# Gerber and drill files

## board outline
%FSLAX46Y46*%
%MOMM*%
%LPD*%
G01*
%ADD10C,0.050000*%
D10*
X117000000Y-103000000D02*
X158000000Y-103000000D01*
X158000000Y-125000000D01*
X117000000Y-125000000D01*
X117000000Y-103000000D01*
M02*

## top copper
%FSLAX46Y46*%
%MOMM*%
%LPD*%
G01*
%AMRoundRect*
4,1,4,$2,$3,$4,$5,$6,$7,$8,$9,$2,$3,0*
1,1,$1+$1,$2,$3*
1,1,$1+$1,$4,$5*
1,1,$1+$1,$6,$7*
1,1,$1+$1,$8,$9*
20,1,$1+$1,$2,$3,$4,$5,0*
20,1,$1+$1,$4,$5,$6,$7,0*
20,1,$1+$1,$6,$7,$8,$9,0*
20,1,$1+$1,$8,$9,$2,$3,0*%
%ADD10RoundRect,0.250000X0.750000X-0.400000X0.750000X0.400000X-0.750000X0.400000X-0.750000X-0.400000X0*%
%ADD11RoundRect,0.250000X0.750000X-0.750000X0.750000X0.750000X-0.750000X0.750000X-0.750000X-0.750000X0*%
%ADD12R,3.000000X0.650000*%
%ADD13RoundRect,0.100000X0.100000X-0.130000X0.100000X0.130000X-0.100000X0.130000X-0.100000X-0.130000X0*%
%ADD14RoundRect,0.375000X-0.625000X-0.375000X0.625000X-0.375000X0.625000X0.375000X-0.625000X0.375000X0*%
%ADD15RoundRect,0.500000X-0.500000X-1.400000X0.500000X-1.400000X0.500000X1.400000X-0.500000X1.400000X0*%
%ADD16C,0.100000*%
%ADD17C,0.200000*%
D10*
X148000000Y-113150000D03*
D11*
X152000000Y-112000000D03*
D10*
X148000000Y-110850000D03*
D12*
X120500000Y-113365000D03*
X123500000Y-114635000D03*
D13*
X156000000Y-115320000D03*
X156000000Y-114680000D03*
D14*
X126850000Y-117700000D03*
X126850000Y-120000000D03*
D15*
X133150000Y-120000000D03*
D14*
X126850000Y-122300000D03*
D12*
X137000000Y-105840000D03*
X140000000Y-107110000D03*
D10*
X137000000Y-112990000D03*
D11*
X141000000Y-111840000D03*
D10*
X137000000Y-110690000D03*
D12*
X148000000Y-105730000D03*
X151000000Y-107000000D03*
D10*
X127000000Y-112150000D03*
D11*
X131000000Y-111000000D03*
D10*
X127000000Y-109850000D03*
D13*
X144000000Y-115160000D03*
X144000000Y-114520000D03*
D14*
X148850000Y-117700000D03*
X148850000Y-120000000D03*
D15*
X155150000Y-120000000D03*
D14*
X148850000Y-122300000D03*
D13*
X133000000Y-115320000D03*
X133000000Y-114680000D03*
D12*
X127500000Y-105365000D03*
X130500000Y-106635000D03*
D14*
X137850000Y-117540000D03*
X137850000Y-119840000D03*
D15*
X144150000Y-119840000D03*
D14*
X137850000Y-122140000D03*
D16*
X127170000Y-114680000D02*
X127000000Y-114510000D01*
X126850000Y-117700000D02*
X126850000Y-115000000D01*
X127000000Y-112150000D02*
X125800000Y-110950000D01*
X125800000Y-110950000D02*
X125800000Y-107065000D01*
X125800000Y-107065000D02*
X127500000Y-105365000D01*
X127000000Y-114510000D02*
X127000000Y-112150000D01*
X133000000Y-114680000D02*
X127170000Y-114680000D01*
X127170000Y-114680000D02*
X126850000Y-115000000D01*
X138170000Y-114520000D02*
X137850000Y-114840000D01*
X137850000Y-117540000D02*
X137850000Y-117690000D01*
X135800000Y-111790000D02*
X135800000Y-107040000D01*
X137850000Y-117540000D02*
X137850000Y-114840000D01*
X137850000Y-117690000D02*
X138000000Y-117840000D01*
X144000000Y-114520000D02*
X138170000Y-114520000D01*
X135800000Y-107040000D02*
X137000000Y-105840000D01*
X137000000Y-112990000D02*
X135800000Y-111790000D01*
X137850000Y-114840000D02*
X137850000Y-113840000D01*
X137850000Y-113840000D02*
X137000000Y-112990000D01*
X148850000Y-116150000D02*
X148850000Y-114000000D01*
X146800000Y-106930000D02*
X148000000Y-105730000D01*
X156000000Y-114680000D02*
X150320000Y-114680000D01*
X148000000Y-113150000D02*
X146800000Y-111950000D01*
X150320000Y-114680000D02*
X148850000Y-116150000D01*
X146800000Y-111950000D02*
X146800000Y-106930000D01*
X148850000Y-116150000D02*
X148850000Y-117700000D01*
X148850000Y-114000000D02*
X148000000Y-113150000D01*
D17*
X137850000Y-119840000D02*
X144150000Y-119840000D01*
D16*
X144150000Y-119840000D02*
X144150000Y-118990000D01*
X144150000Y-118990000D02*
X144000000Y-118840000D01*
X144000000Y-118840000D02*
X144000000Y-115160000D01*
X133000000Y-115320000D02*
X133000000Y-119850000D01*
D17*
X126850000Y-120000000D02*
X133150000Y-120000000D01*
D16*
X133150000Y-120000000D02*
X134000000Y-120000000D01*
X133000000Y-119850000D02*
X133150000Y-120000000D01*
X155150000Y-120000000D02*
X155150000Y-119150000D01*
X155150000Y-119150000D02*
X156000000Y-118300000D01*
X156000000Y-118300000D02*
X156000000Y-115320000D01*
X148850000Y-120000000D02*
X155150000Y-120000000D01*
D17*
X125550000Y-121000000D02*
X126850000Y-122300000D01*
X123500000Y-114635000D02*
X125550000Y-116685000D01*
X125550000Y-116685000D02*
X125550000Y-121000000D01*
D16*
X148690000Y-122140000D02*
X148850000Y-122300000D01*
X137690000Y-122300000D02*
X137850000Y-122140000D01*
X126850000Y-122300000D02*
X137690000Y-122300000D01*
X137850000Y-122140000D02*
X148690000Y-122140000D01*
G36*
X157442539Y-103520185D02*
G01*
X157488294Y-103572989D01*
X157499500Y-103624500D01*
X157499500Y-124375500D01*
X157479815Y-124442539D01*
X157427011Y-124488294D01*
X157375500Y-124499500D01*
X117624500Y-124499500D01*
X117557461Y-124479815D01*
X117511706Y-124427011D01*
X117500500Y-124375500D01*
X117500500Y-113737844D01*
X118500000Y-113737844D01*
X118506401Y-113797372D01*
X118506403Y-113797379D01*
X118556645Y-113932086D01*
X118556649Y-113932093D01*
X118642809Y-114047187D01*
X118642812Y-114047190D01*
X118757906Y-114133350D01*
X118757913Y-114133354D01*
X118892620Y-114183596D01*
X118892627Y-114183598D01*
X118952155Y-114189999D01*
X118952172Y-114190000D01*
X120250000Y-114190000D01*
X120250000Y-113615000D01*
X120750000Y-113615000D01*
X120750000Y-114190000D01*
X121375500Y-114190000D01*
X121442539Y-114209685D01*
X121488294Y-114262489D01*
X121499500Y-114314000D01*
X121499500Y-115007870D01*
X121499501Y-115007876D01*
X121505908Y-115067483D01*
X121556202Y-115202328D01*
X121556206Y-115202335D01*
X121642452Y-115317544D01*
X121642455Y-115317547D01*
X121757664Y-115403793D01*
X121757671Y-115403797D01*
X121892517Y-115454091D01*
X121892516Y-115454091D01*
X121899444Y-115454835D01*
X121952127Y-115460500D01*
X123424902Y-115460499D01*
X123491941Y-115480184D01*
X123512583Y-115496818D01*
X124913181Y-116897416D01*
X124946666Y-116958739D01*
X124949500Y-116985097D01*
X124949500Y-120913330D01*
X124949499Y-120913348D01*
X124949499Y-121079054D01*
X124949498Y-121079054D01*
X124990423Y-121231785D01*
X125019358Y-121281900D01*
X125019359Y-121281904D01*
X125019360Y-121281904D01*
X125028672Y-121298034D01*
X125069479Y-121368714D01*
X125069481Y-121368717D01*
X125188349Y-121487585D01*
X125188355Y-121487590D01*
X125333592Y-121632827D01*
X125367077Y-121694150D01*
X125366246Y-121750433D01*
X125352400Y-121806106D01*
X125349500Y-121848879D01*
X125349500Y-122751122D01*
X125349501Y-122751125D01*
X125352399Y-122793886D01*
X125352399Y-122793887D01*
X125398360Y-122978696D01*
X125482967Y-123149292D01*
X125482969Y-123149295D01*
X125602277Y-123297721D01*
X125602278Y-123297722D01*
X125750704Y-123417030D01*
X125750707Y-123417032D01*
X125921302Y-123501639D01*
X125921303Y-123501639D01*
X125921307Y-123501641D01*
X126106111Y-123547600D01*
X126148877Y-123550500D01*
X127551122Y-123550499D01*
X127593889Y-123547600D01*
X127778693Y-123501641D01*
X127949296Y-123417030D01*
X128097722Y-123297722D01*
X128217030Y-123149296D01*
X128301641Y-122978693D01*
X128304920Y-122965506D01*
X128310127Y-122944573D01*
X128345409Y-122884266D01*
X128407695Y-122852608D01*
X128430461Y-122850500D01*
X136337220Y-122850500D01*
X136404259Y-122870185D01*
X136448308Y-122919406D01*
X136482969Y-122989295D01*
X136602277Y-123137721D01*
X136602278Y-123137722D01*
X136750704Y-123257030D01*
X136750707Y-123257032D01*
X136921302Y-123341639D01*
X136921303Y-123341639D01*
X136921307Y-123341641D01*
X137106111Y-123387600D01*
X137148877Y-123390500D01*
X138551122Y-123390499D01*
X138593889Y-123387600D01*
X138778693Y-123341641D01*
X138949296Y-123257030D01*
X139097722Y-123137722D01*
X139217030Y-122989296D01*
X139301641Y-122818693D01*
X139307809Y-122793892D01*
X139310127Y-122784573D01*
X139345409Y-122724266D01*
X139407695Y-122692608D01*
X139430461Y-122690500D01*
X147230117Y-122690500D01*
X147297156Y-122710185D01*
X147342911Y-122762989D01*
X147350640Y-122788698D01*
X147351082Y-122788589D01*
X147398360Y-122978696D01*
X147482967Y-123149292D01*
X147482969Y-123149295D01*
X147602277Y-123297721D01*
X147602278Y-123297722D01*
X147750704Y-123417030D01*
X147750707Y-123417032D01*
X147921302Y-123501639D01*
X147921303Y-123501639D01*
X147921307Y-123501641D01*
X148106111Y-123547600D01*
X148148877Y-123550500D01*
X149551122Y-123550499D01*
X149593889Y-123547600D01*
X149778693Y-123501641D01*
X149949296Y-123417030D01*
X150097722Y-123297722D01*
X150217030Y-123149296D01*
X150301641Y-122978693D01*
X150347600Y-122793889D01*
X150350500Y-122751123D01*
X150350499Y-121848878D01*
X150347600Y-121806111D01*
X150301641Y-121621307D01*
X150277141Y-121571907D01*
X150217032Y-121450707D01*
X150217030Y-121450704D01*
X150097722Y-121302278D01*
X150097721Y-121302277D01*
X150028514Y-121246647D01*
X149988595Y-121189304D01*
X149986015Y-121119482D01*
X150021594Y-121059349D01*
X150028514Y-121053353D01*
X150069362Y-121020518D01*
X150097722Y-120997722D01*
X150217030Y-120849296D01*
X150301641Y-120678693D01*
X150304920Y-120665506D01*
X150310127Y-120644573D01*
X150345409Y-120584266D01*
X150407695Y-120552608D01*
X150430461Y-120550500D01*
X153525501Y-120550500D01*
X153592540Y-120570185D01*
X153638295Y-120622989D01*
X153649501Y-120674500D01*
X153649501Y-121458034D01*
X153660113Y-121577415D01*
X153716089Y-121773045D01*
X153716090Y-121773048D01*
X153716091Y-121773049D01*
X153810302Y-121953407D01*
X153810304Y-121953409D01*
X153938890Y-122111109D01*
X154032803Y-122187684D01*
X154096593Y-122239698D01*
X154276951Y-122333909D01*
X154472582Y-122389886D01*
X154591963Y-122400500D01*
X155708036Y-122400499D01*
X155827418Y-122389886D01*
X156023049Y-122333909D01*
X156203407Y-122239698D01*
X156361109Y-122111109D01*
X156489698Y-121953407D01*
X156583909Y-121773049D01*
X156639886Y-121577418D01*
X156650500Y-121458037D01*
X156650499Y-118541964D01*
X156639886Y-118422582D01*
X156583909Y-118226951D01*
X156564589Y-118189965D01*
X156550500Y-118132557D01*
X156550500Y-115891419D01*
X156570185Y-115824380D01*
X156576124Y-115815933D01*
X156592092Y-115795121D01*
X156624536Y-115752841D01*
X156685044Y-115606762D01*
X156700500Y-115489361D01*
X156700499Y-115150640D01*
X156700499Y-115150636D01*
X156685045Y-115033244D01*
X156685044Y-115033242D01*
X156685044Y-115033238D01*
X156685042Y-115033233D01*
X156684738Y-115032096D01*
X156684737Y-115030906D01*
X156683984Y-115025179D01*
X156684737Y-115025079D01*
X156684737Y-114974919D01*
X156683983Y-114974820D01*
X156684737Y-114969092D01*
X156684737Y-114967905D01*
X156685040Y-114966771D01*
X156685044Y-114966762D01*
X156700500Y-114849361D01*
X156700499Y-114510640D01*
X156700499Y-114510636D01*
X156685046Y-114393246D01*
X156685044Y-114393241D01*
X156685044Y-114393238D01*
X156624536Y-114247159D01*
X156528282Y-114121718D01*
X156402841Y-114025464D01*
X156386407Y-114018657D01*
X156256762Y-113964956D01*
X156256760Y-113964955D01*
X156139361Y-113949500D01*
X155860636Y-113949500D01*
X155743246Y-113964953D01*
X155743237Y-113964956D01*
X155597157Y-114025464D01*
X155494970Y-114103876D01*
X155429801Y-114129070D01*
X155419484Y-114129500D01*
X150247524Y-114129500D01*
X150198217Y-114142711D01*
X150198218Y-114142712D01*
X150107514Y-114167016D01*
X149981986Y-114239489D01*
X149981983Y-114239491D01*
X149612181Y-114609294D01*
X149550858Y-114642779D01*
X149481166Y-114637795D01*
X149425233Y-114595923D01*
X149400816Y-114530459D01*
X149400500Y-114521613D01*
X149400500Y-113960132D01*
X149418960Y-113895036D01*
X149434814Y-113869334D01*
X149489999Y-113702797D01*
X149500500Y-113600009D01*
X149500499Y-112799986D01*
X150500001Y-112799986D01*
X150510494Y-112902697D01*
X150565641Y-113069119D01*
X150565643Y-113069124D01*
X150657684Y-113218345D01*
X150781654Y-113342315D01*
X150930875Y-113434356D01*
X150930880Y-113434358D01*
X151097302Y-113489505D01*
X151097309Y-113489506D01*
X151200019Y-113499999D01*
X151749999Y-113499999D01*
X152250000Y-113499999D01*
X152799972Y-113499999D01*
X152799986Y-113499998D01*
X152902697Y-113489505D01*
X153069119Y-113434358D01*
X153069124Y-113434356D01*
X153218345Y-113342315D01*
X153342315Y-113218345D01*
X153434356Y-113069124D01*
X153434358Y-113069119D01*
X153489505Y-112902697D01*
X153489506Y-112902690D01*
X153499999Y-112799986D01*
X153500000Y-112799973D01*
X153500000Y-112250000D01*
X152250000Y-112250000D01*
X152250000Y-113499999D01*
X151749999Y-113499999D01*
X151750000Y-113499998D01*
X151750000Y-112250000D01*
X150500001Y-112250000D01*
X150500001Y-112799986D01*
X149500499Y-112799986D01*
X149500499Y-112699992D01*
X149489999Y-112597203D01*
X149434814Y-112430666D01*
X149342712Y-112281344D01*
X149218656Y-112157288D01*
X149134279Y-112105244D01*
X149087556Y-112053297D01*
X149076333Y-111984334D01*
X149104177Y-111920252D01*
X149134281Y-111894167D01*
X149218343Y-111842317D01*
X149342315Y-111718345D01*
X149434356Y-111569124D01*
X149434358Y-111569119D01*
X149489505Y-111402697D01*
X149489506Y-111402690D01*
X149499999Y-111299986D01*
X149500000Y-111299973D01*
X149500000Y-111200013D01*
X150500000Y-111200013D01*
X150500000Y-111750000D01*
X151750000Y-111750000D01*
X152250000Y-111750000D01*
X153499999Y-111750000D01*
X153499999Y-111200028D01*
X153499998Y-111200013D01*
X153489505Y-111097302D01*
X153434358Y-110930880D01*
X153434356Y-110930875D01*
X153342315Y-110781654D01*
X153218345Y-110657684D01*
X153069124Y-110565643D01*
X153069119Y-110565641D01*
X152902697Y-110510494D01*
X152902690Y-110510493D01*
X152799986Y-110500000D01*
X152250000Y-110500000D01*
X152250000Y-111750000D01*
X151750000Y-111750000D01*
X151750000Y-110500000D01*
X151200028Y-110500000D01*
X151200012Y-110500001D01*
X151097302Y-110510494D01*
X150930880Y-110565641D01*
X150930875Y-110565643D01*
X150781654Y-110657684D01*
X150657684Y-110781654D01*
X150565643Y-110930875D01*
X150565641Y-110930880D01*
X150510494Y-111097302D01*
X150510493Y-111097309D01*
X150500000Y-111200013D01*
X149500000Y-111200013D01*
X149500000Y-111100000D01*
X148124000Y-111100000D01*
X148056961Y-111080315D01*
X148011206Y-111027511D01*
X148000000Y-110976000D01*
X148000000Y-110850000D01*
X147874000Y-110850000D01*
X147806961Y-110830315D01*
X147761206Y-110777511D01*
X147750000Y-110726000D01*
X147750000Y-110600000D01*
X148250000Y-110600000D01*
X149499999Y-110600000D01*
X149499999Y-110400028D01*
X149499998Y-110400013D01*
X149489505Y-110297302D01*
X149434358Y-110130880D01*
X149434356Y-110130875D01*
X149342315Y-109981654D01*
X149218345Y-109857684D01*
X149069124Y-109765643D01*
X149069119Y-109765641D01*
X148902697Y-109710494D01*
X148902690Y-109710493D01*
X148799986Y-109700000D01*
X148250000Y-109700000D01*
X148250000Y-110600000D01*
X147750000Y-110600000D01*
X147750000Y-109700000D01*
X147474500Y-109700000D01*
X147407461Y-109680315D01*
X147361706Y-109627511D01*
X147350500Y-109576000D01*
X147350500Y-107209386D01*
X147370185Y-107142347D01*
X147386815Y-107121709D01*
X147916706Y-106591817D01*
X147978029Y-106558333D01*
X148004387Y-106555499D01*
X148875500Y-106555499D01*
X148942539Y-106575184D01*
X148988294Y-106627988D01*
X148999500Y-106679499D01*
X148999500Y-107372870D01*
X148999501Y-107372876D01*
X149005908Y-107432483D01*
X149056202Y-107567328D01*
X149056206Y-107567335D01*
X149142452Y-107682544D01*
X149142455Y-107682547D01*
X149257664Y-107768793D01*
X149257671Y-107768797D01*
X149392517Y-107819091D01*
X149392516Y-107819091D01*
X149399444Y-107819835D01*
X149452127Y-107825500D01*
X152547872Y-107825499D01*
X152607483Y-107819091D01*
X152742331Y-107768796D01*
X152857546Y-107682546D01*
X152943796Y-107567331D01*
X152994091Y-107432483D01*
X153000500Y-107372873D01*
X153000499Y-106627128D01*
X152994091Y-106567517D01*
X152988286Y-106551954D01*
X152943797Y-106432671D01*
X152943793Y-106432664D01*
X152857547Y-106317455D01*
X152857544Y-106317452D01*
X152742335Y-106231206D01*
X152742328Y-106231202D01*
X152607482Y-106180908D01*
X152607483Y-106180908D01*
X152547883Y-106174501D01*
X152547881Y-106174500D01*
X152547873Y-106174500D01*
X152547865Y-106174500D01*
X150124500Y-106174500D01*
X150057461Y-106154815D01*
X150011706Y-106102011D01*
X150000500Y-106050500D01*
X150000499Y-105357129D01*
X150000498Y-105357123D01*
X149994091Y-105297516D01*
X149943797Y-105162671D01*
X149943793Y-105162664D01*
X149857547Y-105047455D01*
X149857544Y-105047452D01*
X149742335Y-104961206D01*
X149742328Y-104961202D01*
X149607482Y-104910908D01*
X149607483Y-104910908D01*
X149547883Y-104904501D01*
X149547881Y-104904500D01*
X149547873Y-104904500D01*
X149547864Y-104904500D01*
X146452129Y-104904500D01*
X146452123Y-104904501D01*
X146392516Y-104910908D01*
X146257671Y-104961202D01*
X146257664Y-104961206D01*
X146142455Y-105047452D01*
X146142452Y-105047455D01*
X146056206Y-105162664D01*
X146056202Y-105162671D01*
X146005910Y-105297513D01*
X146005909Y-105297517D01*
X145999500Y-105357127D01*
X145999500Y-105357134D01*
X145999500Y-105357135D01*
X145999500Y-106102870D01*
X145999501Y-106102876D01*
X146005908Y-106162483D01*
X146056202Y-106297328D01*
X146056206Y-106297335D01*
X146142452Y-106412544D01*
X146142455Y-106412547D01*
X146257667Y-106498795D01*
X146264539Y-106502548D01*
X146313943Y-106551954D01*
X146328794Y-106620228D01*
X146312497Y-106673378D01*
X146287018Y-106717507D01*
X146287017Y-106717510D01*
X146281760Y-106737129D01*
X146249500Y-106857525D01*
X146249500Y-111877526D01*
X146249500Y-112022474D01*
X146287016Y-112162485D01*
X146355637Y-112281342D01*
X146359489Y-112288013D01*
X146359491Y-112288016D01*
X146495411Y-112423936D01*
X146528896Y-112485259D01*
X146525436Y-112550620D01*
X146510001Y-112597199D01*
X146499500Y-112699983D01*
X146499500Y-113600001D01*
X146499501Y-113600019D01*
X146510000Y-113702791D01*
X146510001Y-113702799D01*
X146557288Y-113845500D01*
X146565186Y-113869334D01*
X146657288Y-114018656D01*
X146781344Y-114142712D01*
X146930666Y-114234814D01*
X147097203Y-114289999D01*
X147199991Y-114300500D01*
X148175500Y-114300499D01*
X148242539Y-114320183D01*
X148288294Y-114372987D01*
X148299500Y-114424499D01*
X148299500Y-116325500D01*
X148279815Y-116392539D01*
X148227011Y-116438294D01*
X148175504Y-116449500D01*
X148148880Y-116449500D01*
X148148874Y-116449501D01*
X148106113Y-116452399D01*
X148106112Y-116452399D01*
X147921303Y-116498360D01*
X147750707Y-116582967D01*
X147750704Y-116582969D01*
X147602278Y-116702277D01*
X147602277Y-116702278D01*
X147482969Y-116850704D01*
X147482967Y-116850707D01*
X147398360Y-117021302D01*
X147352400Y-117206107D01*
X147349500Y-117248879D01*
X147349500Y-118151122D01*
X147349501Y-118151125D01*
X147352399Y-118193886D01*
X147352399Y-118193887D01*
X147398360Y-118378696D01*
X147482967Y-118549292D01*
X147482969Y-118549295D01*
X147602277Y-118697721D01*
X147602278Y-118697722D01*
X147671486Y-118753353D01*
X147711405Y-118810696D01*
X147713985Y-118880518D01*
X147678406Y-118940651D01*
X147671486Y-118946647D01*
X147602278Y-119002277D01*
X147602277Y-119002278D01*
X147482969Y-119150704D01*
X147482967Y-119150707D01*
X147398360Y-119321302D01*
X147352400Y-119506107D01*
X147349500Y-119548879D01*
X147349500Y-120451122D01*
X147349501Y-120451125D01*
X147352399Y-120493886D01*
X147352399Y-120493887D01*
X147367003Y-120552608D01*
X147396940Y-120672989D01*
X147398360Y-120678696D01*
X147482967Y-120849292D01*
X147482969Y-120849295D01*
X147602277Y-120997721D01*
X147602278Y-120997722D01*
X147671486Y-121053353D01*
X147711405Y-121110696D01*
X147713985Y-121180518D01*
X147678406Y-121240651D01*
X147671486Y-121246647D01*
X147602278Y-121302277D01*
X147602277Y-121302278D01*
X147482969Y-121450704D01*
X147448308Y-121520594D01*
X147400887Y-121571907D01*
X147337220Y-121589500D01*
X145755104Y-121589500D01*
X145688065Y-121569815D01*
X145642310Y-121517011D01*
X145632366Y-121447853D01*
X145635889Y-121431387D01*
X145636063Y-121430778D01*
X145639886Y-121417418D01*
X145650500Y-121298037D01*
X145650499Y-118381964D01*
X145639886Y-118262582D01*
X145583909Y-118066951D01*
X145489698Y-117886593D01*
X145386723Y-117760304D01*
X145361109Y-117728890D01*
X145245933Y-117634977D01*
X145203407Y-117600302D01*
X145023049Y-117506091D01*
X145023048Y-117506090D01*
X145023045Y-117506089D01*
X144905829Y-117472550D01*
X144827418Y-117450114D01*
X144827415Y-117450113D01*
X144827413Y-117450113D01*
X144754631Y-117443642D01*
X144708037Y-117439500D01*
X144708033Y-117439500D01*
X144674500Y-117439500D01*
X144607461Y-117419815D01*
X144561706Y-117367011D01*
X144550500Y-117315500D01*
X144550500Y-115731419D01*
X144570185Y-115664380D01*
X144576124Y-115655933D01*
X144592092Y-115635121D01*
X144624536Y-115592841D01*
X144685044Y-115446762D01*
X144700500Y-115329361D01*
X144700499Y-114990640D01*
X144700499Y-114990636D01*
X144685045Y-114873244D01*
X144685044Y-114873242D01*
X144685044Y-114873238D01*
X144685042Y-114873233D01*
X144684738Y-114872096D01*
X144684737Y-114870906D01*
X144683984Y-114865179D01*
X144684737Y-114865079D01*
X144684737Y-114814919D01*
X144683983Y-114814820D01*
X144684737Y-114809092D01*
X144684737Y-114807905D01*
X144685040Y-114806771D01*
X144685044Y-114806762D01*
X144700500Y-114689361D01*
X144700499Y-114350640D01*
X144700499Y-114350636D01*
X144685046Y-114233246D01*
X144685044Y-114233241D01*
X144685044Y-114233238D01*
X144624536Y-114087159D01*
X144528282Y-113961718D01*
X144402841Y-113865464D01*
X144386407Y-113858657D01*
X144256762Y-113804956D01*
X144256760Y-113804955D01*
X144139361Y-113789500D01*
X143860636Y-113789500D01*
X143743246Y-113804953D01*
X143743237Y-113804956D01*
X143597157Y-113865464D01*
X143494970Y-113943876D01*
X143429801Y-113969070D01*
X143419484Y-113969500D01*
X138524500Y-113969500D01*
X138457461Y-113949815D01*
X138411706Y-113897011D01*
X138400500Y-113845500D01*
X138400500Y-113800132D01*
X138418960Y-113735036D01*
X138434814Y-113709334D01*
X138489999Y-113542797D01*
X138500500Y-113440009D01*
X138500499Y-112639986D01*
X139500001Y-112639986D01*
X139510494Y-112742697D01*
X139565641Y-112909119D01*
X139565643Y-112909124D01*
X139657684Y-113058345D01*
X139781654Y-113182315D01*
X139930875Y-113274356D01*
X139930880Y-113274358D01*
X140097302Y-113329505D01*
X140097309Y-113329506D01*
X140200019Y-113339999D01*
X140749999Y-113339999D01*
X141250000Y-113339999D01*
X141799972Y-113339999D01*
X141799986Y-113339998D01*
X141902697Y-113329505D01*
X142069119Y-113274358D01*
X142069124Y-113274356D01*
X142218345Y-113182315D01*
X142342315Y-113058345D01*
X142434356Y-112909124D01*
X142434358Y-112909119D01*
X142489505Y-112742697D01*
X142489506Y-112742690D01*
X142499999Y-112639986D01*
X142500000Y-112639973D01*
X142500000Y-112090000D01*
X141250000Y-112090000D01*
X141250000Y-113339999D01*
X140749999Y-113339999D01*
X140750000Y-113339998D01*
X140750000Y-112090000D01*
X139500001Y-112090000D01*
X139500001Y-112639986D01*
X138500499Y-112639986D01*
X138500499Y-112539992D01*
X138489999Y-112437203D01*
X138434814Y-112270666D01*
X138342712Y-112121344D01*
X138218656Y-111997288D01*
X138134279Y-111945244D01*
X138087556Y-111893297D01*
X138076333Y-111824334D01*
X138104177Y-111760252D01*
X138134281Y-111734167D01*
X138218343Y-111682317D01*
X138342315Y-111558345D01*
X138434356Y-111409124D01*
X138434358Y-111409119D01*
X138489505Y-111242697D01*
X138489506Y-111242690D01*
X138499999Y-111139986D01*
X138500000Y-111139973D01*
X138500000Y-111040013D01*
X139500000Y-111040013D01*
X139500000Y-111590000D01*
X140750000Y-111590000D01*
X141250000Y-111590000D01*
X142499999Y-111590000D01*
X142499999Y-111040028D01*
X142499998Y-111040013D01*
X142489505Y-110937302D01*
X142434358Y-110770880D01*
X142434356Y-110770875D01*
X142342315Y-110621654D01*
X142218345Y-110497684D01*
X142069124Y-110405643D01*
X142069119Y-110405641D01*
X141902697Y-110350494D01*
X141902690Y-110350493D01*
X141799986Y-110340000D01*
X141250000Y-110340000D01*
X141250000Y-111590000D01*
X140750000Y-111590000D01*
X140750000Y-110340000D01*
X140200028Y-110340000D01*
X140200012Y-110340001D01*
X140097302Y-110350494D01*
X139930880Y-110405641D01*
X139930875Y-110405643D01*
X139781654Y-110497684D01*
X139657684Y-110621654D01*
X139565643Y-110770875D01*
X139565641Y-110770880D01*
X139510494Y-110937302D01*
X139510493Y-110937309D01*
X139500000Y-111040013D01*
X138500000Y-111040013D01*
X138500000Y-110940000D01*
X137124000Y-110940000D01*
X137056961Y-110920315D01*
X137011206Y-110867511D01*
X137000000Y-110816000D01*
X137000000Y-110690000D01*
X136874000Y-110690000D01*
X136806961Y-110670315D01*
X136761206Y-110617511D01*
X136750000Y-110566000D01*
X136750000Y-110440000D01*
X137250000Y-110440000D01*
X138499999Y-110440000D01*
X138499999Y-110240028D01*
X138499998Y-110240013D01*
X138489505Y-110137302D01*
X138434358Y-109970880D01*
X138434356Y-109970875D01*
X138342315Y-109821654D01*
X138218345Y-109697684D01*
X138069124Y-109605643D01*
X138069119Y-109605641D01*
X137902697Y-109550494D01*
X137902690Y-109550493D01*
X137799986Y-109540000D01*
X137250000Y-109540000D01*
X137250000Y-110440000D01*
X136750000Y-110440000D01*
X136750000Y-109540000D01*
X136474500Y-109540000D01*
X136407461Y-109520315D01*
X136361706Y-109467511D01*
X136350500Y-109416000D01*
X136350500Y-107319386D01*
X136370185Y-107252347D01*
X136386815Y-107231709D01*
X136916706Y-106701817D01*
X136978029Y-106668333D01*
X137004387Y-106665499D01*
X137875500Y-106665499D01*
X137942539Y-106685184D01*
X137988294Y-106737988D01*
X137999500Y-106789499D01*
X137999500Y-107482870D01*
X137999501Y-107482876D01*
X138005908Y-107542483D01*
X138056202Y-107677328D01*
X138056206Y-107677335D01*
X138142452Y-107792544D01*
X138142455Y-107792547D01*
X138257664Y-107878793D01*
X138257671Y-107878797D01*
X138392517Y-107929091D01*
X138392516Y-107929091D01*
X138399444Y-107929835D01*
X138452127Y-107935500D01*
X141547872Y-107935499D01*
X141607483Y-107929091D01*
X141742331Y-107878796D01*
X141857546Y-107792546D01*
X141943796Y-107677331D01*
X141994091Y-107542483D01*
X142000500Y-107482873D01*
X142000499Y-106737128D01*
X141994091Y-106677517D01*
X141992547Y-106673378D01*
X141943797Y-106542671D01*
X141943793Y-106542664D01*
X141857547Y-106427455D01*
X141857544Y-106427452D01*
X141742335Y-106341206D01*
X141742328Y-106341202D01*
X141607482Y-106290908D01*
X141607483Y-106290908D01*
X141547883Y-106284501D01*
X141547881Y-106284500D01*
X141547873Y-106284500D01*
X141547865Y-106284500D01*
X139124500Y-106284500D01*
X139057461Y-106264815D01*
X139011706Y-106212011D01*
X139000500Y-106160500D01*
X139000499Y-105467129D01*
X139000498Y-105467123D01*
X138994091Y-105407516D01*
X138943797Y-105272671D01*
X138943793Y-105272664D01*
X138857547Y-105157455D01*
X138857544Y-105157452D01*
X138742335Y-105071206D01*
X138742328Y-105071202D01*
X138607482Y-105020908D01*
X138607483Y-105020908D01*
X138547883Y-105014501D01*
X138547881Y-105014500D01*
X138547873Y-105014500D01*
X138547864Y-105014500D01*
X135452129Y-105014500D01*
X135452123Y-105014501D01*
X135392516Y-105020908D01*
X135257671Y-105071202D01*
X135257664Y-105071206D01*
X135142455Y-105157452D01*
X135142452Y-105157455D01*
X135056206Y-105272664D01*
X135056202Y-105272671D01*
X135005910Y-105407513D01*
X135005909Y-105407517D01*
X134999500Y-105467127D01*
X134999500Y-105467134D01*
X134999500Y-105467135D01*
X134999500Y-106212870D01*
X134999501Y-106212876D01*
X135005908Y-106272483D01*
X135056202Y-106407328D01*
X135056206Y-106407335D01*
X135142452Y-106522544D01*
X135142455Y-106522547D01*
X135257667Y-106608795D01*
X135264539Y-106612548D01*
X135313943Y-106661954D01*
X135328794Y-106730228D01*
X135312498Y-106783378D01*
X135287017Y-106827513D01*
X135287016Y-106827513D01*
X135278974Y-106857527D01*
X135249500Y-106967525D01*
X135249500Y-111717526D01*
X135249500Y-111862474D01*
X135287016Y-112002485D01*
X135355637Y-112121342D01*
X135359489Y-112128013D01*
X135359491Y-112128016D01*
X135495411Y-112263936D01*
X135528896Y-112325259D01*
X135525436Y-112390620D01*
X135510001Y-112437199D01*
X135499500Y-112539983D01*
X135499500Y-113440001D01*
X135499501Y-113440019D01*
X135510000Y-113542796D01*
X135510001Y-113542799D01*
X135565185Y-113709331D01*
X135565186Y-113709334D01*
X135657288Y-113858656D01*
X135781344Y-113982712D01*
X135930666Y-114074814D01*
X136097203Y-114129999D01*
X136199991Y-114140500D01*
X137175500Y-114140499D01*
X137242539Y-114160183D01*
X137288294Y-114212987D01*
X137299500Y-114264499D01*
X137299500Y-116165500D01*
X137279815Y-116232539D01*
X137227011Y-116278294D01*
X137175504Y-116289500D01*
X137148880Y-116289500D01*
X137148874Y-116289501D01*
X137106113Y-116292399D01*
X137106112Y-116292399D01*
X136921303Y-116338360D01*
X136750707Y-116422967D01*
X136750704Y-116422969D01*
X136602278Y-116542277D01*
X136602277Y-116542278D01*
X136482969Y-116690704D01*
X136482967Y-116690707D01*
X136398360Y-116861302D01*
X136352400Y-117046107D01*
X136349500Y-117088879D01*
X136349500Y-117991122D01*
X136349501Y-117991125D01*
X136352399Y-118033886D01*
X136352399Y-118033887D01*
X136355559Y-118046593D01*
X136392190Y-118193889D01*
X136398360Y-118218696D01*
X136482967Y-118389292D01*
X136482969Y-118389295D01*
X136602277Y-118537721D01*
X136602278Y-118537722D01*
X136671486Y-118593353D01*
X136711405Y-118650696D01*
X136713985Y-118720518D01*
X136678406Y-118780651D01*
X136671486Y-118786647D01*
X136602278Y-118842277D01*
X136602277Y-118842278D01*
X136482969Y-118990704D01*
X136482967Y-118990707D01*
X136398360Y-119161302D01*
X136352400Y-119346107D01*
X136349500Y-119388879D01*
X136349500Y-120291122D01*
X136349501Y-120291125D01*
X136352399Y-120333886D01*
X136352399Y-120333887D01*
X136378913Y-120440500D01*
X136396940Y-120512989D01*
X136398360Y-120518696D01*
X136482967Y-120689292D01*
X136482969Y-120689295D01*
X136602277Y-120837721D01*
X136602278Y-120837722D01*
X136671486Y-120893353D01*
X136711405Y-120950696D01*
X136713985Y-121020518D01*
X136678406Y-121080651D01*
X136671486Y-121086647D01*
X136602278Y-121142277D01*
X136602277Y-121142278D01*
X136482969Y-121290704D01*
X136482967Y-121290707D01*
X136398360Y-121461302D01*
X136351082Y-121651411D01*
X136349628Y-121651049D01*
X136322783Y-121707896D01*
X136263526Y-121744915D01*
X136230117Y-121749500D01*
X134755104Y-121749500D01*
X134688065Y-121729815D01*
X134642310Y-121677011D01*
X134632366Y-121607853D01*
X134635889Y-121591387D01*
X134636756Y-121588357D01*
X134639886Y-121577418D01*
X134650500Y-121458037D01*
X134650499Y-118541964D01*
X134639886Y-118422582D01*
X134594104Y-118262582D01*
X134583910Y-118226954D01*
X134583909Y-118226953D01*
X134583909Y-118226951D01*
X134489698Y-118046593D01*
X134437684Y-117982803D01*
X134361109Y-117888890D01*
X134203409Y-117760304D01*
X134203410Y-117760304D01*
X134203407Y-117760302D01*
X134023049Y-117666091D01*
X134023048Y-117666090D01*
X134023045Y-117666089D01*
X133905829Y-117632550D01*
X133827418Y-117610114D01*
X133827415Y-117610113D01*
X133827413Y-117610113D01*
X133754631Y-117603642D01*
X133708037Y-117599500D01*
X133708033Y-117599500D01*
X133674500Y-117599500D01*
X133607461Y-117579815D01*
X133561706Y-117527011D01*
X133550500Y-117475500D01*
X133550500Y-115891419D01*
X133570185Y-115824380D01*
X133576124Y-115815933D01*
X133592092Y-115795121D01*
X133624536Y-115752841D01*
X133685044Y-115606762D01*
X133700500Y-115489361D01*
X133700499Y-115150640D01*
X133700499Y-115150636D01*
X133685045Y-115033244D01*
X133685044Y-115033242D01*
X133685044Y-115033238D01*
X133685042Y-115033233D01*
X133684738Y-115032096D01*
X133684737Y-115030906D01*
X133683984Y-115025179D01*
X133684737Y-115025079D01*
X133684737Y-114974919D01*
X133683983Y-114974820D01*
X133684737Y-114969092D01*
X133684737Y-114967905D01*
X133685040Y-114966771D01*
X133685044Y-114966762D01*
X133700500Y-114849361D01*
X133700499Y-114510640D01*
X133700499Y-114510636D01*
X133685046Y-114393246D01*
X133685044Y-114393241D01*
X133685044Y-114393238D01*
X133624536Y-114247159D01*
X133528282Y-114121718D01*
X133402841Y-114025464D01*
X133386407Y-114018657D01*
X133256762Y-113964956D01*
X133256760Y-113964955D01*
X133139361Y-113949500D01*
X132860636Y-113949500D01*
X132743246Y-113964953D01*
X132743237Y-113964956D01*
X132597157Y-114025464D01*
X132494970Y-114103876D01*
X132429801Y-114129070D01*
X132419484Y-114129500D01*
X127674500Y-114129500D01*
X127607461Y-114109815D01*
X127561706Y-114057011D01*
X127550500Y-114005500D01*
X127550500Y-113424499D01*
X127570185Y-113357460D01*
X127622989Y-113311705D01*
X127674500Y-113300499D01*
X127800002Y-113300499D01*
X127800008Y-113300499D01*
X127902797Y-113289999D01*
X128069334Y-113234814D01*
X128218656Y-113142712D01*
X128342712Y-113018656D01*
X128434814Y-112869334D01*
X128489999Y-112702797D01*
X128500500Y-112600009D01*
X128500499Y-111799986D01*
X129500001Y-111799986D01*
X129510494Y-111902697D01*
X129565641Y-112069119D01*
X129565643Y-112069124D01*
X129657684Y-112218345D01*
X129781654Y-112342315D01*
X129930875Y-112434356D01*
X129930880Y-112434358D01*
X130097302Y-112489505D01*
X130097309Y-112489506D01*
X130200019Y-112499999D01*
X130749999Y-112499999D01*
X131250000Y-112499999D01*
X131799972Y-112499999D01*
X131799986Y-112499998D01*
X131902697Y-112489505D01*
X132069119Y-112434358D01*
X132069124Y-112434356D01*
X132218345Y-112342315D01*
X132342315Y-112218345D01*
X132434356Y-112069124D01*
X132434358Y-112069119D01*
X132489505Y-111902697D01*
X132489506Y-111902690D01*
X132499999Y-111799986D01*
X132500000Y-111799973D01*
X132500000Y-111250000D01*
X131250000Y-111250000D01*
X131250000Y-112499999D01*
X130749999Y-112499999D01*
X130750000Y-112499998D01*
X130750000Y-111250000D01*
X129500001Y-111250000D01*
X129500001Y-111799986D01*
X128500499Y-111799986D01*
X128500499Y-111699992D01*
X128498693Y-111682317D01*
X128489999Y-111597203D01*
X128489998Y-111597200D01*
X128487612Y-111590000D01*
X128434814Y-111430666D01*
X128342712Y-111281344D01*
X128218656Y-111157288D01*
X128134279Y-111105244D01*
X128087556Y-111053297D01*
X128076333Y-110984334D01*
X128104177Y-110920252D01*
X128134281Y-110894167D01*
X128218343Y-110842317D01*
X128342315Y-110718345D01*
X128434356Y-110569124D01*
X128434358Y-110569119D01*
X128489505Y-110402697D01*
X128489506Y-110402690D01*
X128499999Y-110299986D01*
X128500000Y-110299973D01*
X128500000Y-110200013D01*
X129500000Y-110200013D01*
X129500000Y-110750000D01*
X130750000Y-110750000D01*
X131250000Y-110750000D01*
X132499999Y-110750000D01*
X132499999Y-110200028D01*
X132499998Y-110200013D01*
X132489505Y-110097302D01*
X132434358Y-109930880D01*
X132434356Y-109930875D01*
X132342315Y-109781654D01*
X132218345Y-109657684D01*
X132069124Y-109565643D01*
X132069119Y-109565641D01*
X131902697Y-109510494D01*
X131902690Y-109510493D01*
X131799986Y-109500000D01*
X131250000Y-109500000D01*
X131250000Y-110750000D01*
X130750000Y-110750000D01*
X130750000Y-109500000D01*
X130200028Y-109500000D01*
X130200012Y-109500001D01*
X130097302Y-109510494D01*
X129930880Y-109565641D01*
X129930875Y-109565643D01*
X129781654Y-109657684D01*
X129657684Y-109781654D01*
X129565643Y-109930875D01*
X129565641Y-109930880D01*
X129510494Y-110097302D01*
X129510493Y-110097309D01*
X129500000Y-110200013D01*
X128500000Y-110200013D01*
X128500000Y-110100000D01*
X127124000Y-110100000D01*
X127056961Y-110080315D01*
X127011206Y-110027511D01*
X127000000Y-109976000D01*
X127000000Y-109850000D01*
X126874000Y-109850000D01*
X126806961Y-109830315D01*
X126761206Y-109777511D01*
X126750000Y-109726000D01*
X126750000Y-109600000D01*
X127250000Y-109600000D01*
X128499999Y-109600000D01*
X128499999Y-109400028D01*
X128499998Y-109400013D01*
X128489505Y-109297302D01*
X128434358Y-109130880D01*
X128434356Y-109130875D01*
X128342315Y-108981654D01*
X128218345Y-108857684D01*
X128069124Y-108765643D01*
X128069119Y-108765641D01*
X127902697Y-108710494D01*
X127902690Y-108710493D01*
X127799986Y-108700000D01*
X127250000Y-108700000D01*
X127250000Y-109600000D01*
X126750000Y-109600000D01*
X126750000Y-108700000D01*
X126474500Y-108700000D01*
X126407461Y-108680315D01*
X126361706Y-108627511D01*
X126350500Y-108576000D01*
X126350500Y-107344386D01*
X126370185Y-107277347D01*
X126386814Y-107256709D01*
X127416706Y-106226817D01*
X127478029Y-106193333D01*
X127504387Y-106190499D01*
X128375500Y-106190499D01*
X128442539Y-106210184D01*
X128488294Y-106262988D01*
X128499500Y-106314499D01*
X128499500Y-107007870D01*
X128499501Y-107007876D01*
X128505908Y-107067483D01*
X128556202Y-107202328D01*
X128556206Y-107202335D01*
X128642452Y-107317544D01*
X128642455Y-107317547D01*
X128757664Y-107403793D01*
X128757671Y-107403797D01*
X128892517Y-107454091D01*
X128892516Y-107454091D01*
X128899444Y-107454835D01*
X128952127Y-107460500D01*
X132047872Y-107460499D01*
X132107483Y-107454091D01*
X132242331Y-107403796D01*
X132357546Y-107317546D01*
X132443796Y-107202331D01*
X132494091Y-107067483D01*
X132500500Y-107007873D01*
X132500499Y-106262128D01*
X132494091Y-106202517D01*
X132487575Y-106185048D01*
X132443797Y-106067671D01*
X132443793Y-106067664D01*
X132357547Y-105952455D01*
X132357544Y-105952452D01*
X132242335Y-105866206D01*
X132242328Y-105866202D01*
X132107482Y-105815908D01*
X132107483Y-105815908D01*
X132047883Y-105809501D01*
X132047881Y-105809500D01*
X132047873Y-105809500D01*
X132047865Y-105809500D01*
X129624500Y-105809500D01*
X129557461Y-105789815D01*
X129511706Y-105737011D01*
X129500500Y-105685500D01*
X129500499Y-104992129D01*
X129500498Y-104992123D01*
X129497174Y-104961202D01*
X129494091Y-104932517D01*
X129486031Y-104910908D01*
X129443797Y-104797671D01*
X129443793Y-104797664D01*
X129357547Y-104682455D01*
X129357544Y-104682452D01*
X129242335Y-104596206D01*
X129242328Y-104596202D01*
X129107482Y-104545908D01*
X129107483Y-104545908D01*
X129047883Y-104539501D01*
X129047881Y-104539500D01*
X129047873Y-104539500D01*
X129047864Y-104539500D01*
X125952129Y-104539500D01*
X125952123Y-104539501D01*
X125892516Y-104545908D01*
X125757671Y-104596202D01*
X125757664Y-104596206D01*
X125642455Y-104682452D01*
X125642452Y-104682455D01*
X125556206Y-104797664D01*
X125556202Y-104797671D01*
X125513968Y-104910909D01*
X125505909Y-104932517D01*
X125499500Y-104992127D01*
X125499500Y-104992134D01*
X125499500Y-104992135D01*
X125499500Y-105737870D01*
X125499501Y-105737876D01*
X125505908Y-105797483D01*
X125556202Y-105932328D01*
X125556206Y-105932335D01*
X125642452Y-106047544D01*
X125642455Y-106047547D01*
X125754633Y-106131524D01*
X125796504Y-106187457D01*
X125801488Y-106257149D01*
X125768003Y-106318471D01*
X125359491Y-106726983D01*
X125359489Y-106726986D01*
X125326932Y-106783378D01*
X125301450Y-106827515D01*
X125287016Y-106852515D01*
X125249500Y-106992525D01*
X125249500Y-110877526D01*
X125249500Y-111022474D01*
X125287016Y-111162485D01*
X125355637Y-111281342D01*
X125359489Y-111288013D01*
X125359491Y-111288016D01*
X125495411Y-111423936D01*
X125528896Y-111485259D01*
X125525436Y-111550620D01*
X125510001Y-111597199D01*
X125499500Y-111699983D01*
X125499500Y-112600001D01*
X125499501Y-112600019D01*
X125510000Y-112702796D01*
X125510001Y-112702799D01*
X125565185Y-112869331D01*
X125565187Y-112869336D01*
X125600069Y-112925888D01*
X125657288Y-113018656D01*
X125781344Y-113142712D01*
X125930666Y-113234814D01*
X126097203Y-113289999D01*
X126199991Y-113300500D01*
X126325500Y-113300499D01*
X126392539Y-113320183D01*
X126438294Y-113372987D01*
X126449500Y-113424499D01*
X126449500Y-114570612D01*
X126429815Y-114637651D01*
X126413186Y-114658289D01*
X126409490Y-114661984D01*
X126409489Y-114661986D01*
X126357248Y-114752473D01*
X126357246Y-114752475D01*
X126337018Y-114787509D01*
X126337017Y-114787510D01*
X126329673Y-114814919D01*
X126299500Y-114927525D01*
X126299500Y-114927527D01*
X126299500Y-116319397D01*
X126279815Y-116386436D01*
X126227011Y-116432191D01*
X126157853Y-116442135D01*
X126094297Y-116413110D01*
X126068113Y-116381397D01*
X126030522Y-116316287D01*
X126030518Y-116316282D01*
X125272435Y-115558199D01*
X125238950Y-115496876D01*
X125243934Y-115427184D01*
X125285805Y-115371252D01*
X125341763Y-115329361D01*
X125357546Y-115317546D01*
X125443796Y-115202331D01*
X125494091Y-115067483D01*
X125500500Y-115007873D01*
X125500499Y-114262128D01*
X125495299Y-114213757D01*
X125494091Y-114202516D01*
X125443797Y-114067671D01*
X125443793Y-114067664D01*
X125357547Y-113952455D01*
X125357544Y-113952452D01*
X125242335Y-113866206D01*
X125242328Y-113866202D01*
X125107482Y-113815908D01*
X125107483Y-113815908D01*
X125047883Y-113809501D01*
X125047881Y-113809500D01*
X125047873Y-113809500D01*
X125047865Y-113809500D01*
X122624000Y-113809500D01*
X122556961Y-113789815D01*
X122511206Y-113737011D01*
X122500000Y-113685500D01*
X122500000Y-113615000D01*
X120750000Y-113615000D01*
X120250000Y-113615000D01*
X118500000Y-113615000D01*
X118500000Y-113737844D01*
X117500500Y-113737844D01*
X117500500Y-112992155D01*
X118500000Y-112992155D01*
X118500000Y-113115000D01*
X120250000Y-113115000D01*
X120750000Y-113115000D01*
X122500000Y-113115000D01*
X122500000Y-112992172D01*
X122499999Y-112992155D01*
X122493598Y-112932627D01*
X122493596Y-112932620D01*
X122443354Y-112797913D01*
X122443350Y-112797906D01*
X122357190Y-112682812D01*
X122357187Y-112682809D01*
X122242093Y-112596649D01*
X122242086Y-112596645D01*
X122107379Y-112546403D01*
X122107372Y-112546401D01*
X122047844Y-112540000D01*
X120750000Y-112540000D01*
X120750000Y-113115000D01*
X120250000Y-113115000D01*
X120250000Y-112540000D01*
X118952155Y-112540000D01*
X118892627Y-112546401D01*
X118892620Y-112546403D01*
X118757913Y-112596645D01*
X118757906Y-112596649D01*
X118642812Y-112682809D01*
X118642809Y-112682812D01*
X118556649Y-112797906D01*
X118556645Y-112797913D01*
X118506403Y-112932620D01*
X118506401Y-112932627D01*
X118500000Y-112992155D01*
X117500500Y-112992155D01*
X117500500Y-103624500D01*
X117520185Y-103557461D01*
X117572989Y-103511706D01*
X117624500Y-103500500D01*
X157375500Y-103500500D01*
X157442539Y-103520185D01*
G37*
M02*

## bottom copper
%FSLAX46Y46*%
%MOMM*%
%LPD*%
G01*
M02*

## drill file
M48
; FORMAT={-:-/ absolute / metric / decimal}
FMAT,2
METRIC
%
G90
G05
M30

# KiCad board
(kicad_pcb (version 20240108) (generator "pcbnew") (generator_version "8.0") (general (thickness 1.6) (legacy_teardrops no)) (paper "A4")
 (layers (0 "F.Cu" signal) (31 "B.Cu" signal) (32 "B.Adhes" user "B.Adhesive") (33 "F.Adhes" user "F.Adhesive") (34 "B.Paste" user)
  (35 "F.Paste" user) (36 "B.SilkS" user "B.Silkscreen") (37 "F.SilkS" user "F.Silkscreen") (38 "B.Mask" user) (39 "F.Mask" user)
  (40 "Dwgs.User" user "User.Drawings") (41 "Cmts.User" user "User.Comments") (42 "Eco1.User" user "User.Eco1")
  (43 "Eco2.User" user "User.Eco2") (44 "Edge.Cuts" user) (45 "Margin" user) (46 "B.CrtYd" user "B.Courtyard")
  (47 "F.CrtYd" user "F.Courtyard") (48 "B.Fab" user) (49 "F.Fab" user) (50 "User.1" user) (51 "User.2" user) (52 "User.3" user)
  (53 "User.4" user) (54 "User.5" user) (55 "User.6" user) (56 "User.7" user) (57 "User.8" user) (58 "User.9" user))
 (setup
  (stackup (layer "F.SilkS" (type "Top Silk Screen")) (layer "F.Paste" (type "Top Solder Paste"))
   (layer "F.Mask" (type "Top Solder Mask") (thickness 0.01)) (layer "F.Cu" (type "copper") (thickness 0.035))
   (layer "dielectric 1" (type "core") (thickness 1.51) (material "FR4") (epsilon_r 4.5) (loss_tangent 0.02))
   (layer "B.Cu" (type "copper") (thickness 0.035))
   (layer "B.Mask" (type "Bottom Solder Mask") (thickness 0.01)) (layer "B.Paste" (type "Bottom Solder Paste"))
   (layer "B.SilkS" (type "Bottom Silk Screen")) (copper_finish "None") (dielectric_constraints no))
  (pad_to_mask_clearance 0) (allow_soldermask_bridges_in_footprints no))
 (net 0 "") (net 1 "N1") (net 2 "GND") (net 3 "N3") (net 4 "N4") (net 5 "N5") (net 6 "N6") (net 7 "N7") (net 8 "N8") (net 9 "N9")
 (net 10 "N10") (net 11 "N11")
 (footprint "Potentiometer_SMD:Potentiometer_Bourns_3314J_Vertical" (layer "F.Cu") (at 150 112 90)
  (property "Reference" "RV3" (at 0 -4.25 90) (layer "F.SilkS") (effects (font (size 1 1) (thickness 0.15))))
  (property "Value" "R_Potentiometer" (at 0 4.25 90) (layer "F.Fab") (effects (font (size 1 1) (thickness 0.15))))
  (pad "1" smd roundrect (at -1.15 -2 90) (size 1.3 2) (layers "F.Cu" "F.Paste" "F.Mask") (roundrect_rratio 0.1923076923) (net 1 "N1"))
  (pad "2" smd roundrect (at 0 2 90) (size 2 2) (layers "F.Cu" "F.Paste" "F.Mask") (roundrect_rratio 0.125) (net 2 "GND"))
  (pad "3" smd roundrect (at 1.15 -2 90) (size 1.3 2) (layers "F.Cu" "F.Paste" "F.Mask") (roundrect_rratio 0.1923076923) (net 2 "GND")))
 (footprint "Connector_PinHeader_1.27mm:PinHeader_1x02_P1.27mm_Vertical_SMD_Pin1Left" (layer "F.Cu") (at 122 114)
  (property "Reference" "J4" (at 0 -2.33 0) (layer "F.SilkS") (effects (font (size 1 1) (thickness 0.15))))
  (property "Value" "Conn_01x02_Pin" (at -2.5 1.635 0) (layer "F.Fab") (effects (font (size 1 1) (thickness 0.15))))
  (pad "1" smd rect (at -1.5 -0.635) (size 3 0.65) (layers "F.Cu" "F.Paste" "F.Mask") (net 2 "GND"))
  (pad "2" smd rect (at 1.5 0.635) (size 3 0.65) (layers "F.Cu" "F.Paste" "F.Mask") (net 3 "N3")))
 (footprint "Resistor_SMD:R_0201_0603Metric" (layer "F.Cu") (at 156 115 90)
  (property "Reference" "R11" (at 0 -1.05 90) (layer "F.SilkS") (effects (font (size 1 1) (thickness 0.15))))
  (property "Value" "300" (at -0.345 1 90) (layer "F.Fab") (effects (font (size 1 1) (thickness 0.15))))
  (pad "" smd roundrect (at -0.345 0 90) (size 0.318 0.36) (layers "F.Paste") (roundrect_rratio 0.25))
  (pad "" smd roundrect (at 0.345 0 90) (size 0.318 0.36) (layers "F.Paste") (roundrect_rratio 0.25))
  (pad "1" smd roundrect (at -0.32 0 90) (size 0.46 0.4) (layers "F.Cu" "F.Mask") (roundrect_rratio 0.25) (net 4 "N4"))
  (pad "2" smd roundrect (at 0.32 0 90) (size 0.46 0.4) (layers "F.Cu" "F.Mask") (roundrect_rratio 0.25) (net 1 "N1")))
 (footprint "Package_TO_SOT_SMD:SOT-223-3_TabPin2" (layer "F.Cu") (at 130 120)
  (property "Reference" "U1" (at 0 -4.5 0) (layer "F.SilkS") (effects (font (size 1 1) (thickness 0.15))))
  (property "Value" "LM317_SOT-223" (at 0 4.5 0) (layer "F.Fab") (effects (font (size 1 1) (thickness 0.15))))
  (pad "1" smd roundrect (at -3.15 -2.3) (size 2 1.5) (layers "F.Cu" "F.Paste" "F.Mask") (roundrect_rratio 0.25) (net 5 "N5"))
  (pad "2" smd roundrect (at -3.15 0) (size 2 1.5) (layers "F.Cu" "F.Paste" "F.Mask") (roundrect_rratio 0.25) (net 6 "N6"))
  (pad "2" smd roundrect (at 3.15 0) (size 2 3.8) (layers "F.Cu" "F.Paste" "F.Mask") (roundrect_rratio 0.25) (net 6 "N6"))
  (pad "3" smd roundrect (at -3.15 2.3) (size 2 1.5) (layers "F.Cu" "F.Paste" "F.Mask") (roundrect_rratio 0.25) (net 3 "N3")))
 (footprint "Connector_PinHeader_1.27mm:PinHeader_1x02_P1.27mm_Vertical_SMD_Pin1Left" (layer "F.Cu") (at 138.5 106.475)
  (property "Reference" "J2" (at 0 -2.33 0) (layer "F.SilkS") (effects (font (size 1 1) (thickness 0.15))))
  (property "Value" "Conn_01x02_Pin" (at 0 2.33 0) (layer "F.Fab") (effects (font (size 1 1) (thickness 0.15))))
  (pad "1" smd rect (at -1.5 -0.635) (size 3 0.65) (layers "F.Cu" "F.Paste" "F.Mask") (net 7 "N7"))
  (pad "2" smd rect (at 1.5 0.635) (size 3 0.65) (layers "F.Cu" "F.Paste" "F.Mask") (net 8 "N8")))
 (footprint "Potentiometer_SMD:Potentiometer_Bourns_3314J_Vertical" (layer "F.Cu") (at 139 111.84 90)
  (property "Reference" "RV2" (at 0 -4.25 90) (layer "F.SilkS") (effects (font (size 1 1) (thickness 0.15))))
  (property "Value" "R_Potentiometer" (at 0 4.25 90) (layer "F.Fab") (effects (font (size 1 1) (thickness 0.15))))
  (pad "1" smd roundrect (at -1.15 -2 90) (size 1.3 2) (layers "F.Cu" "F.Paste" "F.Mask") (roundrect_rratio 0.1923076923) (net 7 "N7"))
  (pad "2" smd roundrect (at 0 2 90) (size 2 2) (layers "F.Cu" "F.Paste" "F.Mask") (roundrect_rratio 0.125) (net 2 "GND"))
  (pad "3" smd roundrect (at 1.15 -2 90) (size 1.3 2) (layers "F.Cu" "F.Paste" "F.Mask") (roundrect_rratio 0.1923076923) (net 2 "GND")))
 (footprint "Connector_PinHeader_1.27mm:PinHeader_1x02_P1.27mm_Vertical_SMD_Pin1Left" (layer "F.Cu") (at 149.5 106.365)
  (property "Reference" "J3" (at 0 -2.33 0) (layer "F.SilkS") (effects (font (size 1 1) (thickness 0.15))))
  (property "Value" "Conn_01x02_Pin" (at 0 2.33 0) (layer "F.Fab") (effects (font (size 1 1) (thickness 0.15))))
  (pad "1" smd rect (at -1.5 -0.635) (size 3 0.65) (layers "F.Cu" "F.Paste" "F.Mask") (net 1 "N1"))
  (pad "2" smd rect (at 1.5 0.635) (size 3 0.65) (layers "F.Cu" "F.Paste" "F.Mask") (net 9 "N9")))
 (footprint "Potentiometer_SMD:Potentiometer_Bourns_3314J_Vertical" (layer "F.Cu") (at 129 111 90)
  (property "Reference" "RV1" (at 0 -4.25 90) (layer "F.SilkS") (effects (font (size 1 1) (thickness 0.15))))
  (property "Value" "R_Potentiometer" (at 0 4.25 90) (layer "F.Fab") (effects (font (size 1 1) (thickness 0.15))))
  (pad "1" smd roundrect (at -1.15 -2 90) (size 1.3 2) (layers "F.Cu" "F.Paste" "F.Mask") (roundrect_rratio 0.1923076923) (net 5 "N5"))
  (pad "2" smd roundrect (at 0 2 90) (size 2 2) (layers "F.Cu" "F.Paste" "F.Mask") (roundrect_rratio 0.125) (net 2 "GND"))
  (pad "3" smd roundrect (at 1.15 -2 90) (size 1.3 2) (layers "F.Cu" "F.Paste" "F.Mask") (roundrect_rratio 0.1923076923) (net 2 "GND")))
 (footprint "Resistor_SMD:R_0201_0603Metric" (layer "F.Cu") (at 144 114.84 90)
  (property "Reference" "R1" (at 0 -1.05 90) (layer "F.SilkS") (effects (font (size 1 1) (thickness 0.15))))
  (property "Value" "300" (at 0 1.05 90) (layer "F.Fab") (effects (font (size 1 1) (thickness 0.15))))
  (pad "" smd roundrect (at -0.345 0 90) (size 0.318 0.36) (layers "F.Paste") (roundrect_rratio 0.25))
  (pad "" smd roundrect (at 0.345 0 90) (size 0.318 0.36) (layers "F.Paste") (roundrect_rratio 0.25))
  (pad "1" smd roundrect (at -0.32 0 90) (size 0.46 0.4) (layers "F.Cu" "F.Mask") (roundrect_rratio 0.25) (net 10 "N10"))
  (pad "2" smd roundrect (at 0.32 0 90) (size 0.46 0.4) (layers "F.Cu" "F.Mask") (roundrect_rratio 0.25) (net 7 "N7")))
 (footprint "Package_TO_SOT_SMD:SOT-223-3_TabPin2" (layer "F.Cu") (at 152 120)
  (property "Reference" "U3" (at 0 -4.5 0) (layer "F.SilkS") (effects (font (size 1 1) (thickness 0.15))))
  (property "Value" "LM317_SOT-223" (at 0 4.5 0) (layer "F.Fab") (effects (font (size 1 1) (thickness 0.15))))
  (pad "1" smd roundrect (at -3.15 -2.3) (size 2 1.5) (layers "F.Cu" "F.Paste" "F.Mask") (roundrect_rratio 0.25) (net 1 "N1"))
  (pad "2" smd roundrect (at -3.15 0) (size 2 1.5) (layers "F.Cu" "F.Paste" "F.Mask") (roundrect_rratio 0.25) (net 4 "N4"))
  (pad "2" smd roundrect (at 3.15 0) (size 2 3.8) (layers "F.Cu" "F.Paste" "F.Mask") (roundrect_rratio 0.25) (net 4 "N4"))
  (pad "3" smd roundrect (at -3.15 2.3) (size 2 1.5) (layers "F.Cu" "F.Paste" "F.Mask") (roundrect_rratio 0.25) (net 3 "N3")))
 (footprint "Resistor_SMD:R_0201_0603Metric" (layer "F.Cu") (at 133 115 90)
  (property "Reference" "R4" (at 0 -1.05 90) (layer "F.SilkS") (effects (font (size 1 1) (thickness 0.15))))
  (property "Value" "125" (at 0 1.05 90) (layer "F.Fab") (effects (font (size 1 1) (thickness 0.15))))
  (pad "" smd roundrect (at -0.345 0 90) (size 0.318 0.36) (layers "F.Paste") (roundrect_rratio 0.25))
  (pad "" smd roundrect (at 0.345 0 90) (size 0.318 0.36) (layers "F.Paste") (roundrect_rratio 0.25))
  (pad "1" smd roundrect (at -0.32 0 90) (size 0.46 0.4) (layers "F.Cu" "F.Mask") (roundrect_rratio 0.25) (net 6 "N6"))
  (pad "2" smd roundrect (at 0.32 0 90) (size 0.46 0.4) (layers "F.Cu" "F.Mask") (roundrect_rratio 0.25) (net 5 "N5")))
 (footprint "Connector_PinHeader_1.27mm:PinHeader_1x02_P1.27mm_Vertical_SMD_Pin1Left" (layer "F.Cu") (at 129 106)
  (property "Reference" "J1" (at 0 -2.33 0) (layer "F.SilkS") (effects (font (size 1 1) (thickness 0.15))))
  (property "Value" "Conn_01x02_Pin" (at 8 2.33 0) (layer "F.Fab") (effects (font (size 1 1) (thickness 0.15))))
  (pad "1" smd rect (at -1.5 -0.635) (size 3 0.65) (layers "F.Cu" "F.Paste" "F.Mask") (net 5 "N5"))
  (pad "2" smd rect (at 1.5 0.635) (size 3 0.65) (layers "F.Cu" "F.Paste" "F.Mask") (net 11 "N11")))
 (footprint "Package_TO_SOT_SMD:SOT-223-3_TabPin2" (layer "F.Cu") (at 141 119.84)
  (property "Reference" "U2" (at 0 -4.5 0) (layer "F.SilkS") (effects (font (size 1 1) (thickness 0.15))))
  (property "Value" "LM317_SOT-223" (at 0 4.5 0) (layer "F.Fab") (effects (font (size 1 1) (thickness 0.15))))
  (pad "1" smd roundrect (at -3.15 -2.3) (size 2 1.5) (layers "F.Cu" "F.Paste" "F.Mask") (roundrect_rratio 0.25) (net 7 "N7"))
  (pad "2" smd roundrect (at -3.15 0) (size 2 1.5) (layers "F.Cu" "F.Paste" "F.Mask") (roundrect_rratio 0.25) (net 10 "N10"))
  (pad "2" smd roundrect (at 3.15 0) (size 2 3.8) (layers "F.Cu" "F.Paste" "F.Mask") (roundrect_rratio 0.25) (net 10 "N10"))
  (pad "3" smd roundrect (at -3.15 2.3) (size 2 1.5) (layers "F.Cu" "F.Paste" "F.Mask") (roundrect_rratio 0.25) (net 3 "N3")))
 (gr_rect (start 117 103) (end 158 125) (stroke (width 0.05) (type default)) (fill none) (layer "Edge.Cuts"))
 (segment (start 127.17 114.68) (end 127 114.51) (width 0.1) (layer "F.Cu") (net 5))
 (segment (start 126.85 117.7) (end 126.85 115) (width 0.1) (layer "F.Cu") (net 5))
 (segment (start 127 112.15) (end 125.8 110.95) (width 0.1) (layer "F.Cu") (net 5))
 (segment (start 125.8 110.95) (end 125.8 107.065) (width 0.1) (layer "F.Cu") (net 5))
 (segment (start 125.8 107.065) (end 127.5 105.365) (width 0.1) (layer "F.Cu") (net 5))
 (segment (start 127 114.51) (end 127 112.15) (width 0.1) (layer "F.Cu") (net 5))
 (segment (start 133 114.68) (end 127.17 114.68) (width 0.1) (layer "F.Cu") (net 5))
 (segment (start 127.17 114.68) (end 126.85 115) (width 0.1) (layer "F.Cu") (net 5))
 (segment (start 138.17 114.52) (end 137.85 114.84) (width 0.1) (layer "F.Cu") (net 7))
 (segment (start 137.85 117.54) (end 137.85 117.69) (width 0.1) (layer "F.Cu") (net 7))
 (segment (start 135.8 111.79) (end 135.8 107.04) (width 0.1) (layer "F.Cu") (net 7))
 (segment (start 137.85 117.54) (end 137.85 114.84) (width 0.1) (layer "F.Cu") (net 7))
 (segment (start 137.85 117.69) (end 138 117.84) (width 0.1) (layer "F.Cu") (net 7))
 (segment (start 144 114.52) (end 138.17 114.52) (width 0.1) (layer "F.Cu") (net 7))
 (segment (start 135.8 107.04) (end 137 105.84) (width 0.1) (layer "F.Cu") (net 7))
 (segment (start 137 112.99) (end 135.8 111.79) (width 0.1) (layer "F.Cu") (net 7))
 (segment (start 137.85 114.84) (end 137.85 113.84) (width 0.1) (layer "F.Cu") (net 7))
 (segment (start 137.85 113.84) (end 137 112.99) (width 0.1) (layer "F.Cu") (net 7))
 (segment (start 148.85 116.15) (end 148.85 114) (width 0.1) (layer "F.Cu") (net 1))
 (segment (start 146.8 106.93) (end 148 105.73) (width 0.1) (layer "F.Cu") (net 1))
 (segment (start 156 114.68) (end 150.32 114.68) (width 0.1) (layer "F.Cu") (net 1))
 (segment (start 148 113.15) (end 146.8 111.95) (width 0.1) (layer "F.Cu") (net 1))
 (segment (start 150.32 114.68) (end 148.85 116.15) (width 0.1) (layer "F.Cu") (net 1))
 (segment (start 146.8 111.95) (end 146.8 106.93) (width 0.1) (layer "F.Cu") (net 1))
 (segment (start 148.85 116.15) (end 148.85 117.7) (width 0.1) (layer "F.Cu") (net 1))
 (segment (start 148.85 114) (end 148 113.15) (width 0.1) (layer "F.Cu") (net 1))
 (segment (start 137.85 119.84) (end 144.15 119.84) (width 0.2) (layer "F.Cu") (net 10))
 (segment (start 144.15 119.84) (end 144.15 118.99) (width 0.1) (layer "F.Cu") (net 10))
 (segment (start 144.15 118.99) (end 144 118.84) (width 0.1) (layer "F.Cu") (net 10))
 (segment (start 144 118.84) (end 144 115.16) (width 0.1) (layer "F.Cu") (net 10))
 (segment (start 133 115.32) (end 133 119.85) (width 0.1) (layer "F.Cu") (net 6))
 (segment (start 126.85 120) (end 133.15 120) (width 0.2) (layer "F.Cu") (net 6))
 (segment (start 133.15 120) (end 134 120) (width 0.1) (layer "F.Cu") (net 6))
 (segment (start 133 119.85) (end 133.15 120) (width 0.1) (layer "F.Cu") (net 6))
 (segment (start 155.15 120) (end 155.15 119.15) (width 0.1) (layer "F.Cu") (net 4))
 (segment (start 155.15 119.15) (end 156 118.3) (width 0.1) (layer "F.Cu") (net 4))
 (segment (start 156 118.3) (end 156 115.32) (width 0.1) (layer "F.Cu") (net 4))
 (segment (start 148.85 120) (end 155.15 120) (width 0.1) (layer "F.Cu") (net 4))
 (segment (start 125.55 121) (end 126.85 122.3) (width 0.2) (layer "F.Cu") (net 3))
 (segment (start 123.5 114.635) (end 125.55 116.685) (width 0.2) (layer "F.Cu") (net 3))
 (segment (start 125.55 116.685) (end 125.55 121) (width 0.2) (layer "F.Cu") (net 3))
 (segment (start 148.69 122.14) (end 148.85 122.3) (width 0.1) (layer "F.Cu") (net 3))
 (segment (start 137.69 122.3) (end 137.85 122.14) (width 0.1) (layer "F.Cu") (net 3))
 (segment (start 126.85 122.3) (end 137.69 122.3) (width 0.1) (layer "F.Cu") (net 3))
 (segment (start 137.85 122.14) (end 148.69 122.14) (width 0.1) (layer "F.Cu") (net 3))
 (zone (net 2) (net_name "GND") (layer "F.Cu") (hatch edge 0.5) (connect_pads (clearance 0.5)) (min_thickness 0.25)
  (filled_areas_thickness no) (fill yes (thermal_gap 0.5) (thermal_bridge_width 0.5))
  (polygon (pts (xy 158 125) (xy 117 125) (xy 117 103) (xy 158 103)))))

